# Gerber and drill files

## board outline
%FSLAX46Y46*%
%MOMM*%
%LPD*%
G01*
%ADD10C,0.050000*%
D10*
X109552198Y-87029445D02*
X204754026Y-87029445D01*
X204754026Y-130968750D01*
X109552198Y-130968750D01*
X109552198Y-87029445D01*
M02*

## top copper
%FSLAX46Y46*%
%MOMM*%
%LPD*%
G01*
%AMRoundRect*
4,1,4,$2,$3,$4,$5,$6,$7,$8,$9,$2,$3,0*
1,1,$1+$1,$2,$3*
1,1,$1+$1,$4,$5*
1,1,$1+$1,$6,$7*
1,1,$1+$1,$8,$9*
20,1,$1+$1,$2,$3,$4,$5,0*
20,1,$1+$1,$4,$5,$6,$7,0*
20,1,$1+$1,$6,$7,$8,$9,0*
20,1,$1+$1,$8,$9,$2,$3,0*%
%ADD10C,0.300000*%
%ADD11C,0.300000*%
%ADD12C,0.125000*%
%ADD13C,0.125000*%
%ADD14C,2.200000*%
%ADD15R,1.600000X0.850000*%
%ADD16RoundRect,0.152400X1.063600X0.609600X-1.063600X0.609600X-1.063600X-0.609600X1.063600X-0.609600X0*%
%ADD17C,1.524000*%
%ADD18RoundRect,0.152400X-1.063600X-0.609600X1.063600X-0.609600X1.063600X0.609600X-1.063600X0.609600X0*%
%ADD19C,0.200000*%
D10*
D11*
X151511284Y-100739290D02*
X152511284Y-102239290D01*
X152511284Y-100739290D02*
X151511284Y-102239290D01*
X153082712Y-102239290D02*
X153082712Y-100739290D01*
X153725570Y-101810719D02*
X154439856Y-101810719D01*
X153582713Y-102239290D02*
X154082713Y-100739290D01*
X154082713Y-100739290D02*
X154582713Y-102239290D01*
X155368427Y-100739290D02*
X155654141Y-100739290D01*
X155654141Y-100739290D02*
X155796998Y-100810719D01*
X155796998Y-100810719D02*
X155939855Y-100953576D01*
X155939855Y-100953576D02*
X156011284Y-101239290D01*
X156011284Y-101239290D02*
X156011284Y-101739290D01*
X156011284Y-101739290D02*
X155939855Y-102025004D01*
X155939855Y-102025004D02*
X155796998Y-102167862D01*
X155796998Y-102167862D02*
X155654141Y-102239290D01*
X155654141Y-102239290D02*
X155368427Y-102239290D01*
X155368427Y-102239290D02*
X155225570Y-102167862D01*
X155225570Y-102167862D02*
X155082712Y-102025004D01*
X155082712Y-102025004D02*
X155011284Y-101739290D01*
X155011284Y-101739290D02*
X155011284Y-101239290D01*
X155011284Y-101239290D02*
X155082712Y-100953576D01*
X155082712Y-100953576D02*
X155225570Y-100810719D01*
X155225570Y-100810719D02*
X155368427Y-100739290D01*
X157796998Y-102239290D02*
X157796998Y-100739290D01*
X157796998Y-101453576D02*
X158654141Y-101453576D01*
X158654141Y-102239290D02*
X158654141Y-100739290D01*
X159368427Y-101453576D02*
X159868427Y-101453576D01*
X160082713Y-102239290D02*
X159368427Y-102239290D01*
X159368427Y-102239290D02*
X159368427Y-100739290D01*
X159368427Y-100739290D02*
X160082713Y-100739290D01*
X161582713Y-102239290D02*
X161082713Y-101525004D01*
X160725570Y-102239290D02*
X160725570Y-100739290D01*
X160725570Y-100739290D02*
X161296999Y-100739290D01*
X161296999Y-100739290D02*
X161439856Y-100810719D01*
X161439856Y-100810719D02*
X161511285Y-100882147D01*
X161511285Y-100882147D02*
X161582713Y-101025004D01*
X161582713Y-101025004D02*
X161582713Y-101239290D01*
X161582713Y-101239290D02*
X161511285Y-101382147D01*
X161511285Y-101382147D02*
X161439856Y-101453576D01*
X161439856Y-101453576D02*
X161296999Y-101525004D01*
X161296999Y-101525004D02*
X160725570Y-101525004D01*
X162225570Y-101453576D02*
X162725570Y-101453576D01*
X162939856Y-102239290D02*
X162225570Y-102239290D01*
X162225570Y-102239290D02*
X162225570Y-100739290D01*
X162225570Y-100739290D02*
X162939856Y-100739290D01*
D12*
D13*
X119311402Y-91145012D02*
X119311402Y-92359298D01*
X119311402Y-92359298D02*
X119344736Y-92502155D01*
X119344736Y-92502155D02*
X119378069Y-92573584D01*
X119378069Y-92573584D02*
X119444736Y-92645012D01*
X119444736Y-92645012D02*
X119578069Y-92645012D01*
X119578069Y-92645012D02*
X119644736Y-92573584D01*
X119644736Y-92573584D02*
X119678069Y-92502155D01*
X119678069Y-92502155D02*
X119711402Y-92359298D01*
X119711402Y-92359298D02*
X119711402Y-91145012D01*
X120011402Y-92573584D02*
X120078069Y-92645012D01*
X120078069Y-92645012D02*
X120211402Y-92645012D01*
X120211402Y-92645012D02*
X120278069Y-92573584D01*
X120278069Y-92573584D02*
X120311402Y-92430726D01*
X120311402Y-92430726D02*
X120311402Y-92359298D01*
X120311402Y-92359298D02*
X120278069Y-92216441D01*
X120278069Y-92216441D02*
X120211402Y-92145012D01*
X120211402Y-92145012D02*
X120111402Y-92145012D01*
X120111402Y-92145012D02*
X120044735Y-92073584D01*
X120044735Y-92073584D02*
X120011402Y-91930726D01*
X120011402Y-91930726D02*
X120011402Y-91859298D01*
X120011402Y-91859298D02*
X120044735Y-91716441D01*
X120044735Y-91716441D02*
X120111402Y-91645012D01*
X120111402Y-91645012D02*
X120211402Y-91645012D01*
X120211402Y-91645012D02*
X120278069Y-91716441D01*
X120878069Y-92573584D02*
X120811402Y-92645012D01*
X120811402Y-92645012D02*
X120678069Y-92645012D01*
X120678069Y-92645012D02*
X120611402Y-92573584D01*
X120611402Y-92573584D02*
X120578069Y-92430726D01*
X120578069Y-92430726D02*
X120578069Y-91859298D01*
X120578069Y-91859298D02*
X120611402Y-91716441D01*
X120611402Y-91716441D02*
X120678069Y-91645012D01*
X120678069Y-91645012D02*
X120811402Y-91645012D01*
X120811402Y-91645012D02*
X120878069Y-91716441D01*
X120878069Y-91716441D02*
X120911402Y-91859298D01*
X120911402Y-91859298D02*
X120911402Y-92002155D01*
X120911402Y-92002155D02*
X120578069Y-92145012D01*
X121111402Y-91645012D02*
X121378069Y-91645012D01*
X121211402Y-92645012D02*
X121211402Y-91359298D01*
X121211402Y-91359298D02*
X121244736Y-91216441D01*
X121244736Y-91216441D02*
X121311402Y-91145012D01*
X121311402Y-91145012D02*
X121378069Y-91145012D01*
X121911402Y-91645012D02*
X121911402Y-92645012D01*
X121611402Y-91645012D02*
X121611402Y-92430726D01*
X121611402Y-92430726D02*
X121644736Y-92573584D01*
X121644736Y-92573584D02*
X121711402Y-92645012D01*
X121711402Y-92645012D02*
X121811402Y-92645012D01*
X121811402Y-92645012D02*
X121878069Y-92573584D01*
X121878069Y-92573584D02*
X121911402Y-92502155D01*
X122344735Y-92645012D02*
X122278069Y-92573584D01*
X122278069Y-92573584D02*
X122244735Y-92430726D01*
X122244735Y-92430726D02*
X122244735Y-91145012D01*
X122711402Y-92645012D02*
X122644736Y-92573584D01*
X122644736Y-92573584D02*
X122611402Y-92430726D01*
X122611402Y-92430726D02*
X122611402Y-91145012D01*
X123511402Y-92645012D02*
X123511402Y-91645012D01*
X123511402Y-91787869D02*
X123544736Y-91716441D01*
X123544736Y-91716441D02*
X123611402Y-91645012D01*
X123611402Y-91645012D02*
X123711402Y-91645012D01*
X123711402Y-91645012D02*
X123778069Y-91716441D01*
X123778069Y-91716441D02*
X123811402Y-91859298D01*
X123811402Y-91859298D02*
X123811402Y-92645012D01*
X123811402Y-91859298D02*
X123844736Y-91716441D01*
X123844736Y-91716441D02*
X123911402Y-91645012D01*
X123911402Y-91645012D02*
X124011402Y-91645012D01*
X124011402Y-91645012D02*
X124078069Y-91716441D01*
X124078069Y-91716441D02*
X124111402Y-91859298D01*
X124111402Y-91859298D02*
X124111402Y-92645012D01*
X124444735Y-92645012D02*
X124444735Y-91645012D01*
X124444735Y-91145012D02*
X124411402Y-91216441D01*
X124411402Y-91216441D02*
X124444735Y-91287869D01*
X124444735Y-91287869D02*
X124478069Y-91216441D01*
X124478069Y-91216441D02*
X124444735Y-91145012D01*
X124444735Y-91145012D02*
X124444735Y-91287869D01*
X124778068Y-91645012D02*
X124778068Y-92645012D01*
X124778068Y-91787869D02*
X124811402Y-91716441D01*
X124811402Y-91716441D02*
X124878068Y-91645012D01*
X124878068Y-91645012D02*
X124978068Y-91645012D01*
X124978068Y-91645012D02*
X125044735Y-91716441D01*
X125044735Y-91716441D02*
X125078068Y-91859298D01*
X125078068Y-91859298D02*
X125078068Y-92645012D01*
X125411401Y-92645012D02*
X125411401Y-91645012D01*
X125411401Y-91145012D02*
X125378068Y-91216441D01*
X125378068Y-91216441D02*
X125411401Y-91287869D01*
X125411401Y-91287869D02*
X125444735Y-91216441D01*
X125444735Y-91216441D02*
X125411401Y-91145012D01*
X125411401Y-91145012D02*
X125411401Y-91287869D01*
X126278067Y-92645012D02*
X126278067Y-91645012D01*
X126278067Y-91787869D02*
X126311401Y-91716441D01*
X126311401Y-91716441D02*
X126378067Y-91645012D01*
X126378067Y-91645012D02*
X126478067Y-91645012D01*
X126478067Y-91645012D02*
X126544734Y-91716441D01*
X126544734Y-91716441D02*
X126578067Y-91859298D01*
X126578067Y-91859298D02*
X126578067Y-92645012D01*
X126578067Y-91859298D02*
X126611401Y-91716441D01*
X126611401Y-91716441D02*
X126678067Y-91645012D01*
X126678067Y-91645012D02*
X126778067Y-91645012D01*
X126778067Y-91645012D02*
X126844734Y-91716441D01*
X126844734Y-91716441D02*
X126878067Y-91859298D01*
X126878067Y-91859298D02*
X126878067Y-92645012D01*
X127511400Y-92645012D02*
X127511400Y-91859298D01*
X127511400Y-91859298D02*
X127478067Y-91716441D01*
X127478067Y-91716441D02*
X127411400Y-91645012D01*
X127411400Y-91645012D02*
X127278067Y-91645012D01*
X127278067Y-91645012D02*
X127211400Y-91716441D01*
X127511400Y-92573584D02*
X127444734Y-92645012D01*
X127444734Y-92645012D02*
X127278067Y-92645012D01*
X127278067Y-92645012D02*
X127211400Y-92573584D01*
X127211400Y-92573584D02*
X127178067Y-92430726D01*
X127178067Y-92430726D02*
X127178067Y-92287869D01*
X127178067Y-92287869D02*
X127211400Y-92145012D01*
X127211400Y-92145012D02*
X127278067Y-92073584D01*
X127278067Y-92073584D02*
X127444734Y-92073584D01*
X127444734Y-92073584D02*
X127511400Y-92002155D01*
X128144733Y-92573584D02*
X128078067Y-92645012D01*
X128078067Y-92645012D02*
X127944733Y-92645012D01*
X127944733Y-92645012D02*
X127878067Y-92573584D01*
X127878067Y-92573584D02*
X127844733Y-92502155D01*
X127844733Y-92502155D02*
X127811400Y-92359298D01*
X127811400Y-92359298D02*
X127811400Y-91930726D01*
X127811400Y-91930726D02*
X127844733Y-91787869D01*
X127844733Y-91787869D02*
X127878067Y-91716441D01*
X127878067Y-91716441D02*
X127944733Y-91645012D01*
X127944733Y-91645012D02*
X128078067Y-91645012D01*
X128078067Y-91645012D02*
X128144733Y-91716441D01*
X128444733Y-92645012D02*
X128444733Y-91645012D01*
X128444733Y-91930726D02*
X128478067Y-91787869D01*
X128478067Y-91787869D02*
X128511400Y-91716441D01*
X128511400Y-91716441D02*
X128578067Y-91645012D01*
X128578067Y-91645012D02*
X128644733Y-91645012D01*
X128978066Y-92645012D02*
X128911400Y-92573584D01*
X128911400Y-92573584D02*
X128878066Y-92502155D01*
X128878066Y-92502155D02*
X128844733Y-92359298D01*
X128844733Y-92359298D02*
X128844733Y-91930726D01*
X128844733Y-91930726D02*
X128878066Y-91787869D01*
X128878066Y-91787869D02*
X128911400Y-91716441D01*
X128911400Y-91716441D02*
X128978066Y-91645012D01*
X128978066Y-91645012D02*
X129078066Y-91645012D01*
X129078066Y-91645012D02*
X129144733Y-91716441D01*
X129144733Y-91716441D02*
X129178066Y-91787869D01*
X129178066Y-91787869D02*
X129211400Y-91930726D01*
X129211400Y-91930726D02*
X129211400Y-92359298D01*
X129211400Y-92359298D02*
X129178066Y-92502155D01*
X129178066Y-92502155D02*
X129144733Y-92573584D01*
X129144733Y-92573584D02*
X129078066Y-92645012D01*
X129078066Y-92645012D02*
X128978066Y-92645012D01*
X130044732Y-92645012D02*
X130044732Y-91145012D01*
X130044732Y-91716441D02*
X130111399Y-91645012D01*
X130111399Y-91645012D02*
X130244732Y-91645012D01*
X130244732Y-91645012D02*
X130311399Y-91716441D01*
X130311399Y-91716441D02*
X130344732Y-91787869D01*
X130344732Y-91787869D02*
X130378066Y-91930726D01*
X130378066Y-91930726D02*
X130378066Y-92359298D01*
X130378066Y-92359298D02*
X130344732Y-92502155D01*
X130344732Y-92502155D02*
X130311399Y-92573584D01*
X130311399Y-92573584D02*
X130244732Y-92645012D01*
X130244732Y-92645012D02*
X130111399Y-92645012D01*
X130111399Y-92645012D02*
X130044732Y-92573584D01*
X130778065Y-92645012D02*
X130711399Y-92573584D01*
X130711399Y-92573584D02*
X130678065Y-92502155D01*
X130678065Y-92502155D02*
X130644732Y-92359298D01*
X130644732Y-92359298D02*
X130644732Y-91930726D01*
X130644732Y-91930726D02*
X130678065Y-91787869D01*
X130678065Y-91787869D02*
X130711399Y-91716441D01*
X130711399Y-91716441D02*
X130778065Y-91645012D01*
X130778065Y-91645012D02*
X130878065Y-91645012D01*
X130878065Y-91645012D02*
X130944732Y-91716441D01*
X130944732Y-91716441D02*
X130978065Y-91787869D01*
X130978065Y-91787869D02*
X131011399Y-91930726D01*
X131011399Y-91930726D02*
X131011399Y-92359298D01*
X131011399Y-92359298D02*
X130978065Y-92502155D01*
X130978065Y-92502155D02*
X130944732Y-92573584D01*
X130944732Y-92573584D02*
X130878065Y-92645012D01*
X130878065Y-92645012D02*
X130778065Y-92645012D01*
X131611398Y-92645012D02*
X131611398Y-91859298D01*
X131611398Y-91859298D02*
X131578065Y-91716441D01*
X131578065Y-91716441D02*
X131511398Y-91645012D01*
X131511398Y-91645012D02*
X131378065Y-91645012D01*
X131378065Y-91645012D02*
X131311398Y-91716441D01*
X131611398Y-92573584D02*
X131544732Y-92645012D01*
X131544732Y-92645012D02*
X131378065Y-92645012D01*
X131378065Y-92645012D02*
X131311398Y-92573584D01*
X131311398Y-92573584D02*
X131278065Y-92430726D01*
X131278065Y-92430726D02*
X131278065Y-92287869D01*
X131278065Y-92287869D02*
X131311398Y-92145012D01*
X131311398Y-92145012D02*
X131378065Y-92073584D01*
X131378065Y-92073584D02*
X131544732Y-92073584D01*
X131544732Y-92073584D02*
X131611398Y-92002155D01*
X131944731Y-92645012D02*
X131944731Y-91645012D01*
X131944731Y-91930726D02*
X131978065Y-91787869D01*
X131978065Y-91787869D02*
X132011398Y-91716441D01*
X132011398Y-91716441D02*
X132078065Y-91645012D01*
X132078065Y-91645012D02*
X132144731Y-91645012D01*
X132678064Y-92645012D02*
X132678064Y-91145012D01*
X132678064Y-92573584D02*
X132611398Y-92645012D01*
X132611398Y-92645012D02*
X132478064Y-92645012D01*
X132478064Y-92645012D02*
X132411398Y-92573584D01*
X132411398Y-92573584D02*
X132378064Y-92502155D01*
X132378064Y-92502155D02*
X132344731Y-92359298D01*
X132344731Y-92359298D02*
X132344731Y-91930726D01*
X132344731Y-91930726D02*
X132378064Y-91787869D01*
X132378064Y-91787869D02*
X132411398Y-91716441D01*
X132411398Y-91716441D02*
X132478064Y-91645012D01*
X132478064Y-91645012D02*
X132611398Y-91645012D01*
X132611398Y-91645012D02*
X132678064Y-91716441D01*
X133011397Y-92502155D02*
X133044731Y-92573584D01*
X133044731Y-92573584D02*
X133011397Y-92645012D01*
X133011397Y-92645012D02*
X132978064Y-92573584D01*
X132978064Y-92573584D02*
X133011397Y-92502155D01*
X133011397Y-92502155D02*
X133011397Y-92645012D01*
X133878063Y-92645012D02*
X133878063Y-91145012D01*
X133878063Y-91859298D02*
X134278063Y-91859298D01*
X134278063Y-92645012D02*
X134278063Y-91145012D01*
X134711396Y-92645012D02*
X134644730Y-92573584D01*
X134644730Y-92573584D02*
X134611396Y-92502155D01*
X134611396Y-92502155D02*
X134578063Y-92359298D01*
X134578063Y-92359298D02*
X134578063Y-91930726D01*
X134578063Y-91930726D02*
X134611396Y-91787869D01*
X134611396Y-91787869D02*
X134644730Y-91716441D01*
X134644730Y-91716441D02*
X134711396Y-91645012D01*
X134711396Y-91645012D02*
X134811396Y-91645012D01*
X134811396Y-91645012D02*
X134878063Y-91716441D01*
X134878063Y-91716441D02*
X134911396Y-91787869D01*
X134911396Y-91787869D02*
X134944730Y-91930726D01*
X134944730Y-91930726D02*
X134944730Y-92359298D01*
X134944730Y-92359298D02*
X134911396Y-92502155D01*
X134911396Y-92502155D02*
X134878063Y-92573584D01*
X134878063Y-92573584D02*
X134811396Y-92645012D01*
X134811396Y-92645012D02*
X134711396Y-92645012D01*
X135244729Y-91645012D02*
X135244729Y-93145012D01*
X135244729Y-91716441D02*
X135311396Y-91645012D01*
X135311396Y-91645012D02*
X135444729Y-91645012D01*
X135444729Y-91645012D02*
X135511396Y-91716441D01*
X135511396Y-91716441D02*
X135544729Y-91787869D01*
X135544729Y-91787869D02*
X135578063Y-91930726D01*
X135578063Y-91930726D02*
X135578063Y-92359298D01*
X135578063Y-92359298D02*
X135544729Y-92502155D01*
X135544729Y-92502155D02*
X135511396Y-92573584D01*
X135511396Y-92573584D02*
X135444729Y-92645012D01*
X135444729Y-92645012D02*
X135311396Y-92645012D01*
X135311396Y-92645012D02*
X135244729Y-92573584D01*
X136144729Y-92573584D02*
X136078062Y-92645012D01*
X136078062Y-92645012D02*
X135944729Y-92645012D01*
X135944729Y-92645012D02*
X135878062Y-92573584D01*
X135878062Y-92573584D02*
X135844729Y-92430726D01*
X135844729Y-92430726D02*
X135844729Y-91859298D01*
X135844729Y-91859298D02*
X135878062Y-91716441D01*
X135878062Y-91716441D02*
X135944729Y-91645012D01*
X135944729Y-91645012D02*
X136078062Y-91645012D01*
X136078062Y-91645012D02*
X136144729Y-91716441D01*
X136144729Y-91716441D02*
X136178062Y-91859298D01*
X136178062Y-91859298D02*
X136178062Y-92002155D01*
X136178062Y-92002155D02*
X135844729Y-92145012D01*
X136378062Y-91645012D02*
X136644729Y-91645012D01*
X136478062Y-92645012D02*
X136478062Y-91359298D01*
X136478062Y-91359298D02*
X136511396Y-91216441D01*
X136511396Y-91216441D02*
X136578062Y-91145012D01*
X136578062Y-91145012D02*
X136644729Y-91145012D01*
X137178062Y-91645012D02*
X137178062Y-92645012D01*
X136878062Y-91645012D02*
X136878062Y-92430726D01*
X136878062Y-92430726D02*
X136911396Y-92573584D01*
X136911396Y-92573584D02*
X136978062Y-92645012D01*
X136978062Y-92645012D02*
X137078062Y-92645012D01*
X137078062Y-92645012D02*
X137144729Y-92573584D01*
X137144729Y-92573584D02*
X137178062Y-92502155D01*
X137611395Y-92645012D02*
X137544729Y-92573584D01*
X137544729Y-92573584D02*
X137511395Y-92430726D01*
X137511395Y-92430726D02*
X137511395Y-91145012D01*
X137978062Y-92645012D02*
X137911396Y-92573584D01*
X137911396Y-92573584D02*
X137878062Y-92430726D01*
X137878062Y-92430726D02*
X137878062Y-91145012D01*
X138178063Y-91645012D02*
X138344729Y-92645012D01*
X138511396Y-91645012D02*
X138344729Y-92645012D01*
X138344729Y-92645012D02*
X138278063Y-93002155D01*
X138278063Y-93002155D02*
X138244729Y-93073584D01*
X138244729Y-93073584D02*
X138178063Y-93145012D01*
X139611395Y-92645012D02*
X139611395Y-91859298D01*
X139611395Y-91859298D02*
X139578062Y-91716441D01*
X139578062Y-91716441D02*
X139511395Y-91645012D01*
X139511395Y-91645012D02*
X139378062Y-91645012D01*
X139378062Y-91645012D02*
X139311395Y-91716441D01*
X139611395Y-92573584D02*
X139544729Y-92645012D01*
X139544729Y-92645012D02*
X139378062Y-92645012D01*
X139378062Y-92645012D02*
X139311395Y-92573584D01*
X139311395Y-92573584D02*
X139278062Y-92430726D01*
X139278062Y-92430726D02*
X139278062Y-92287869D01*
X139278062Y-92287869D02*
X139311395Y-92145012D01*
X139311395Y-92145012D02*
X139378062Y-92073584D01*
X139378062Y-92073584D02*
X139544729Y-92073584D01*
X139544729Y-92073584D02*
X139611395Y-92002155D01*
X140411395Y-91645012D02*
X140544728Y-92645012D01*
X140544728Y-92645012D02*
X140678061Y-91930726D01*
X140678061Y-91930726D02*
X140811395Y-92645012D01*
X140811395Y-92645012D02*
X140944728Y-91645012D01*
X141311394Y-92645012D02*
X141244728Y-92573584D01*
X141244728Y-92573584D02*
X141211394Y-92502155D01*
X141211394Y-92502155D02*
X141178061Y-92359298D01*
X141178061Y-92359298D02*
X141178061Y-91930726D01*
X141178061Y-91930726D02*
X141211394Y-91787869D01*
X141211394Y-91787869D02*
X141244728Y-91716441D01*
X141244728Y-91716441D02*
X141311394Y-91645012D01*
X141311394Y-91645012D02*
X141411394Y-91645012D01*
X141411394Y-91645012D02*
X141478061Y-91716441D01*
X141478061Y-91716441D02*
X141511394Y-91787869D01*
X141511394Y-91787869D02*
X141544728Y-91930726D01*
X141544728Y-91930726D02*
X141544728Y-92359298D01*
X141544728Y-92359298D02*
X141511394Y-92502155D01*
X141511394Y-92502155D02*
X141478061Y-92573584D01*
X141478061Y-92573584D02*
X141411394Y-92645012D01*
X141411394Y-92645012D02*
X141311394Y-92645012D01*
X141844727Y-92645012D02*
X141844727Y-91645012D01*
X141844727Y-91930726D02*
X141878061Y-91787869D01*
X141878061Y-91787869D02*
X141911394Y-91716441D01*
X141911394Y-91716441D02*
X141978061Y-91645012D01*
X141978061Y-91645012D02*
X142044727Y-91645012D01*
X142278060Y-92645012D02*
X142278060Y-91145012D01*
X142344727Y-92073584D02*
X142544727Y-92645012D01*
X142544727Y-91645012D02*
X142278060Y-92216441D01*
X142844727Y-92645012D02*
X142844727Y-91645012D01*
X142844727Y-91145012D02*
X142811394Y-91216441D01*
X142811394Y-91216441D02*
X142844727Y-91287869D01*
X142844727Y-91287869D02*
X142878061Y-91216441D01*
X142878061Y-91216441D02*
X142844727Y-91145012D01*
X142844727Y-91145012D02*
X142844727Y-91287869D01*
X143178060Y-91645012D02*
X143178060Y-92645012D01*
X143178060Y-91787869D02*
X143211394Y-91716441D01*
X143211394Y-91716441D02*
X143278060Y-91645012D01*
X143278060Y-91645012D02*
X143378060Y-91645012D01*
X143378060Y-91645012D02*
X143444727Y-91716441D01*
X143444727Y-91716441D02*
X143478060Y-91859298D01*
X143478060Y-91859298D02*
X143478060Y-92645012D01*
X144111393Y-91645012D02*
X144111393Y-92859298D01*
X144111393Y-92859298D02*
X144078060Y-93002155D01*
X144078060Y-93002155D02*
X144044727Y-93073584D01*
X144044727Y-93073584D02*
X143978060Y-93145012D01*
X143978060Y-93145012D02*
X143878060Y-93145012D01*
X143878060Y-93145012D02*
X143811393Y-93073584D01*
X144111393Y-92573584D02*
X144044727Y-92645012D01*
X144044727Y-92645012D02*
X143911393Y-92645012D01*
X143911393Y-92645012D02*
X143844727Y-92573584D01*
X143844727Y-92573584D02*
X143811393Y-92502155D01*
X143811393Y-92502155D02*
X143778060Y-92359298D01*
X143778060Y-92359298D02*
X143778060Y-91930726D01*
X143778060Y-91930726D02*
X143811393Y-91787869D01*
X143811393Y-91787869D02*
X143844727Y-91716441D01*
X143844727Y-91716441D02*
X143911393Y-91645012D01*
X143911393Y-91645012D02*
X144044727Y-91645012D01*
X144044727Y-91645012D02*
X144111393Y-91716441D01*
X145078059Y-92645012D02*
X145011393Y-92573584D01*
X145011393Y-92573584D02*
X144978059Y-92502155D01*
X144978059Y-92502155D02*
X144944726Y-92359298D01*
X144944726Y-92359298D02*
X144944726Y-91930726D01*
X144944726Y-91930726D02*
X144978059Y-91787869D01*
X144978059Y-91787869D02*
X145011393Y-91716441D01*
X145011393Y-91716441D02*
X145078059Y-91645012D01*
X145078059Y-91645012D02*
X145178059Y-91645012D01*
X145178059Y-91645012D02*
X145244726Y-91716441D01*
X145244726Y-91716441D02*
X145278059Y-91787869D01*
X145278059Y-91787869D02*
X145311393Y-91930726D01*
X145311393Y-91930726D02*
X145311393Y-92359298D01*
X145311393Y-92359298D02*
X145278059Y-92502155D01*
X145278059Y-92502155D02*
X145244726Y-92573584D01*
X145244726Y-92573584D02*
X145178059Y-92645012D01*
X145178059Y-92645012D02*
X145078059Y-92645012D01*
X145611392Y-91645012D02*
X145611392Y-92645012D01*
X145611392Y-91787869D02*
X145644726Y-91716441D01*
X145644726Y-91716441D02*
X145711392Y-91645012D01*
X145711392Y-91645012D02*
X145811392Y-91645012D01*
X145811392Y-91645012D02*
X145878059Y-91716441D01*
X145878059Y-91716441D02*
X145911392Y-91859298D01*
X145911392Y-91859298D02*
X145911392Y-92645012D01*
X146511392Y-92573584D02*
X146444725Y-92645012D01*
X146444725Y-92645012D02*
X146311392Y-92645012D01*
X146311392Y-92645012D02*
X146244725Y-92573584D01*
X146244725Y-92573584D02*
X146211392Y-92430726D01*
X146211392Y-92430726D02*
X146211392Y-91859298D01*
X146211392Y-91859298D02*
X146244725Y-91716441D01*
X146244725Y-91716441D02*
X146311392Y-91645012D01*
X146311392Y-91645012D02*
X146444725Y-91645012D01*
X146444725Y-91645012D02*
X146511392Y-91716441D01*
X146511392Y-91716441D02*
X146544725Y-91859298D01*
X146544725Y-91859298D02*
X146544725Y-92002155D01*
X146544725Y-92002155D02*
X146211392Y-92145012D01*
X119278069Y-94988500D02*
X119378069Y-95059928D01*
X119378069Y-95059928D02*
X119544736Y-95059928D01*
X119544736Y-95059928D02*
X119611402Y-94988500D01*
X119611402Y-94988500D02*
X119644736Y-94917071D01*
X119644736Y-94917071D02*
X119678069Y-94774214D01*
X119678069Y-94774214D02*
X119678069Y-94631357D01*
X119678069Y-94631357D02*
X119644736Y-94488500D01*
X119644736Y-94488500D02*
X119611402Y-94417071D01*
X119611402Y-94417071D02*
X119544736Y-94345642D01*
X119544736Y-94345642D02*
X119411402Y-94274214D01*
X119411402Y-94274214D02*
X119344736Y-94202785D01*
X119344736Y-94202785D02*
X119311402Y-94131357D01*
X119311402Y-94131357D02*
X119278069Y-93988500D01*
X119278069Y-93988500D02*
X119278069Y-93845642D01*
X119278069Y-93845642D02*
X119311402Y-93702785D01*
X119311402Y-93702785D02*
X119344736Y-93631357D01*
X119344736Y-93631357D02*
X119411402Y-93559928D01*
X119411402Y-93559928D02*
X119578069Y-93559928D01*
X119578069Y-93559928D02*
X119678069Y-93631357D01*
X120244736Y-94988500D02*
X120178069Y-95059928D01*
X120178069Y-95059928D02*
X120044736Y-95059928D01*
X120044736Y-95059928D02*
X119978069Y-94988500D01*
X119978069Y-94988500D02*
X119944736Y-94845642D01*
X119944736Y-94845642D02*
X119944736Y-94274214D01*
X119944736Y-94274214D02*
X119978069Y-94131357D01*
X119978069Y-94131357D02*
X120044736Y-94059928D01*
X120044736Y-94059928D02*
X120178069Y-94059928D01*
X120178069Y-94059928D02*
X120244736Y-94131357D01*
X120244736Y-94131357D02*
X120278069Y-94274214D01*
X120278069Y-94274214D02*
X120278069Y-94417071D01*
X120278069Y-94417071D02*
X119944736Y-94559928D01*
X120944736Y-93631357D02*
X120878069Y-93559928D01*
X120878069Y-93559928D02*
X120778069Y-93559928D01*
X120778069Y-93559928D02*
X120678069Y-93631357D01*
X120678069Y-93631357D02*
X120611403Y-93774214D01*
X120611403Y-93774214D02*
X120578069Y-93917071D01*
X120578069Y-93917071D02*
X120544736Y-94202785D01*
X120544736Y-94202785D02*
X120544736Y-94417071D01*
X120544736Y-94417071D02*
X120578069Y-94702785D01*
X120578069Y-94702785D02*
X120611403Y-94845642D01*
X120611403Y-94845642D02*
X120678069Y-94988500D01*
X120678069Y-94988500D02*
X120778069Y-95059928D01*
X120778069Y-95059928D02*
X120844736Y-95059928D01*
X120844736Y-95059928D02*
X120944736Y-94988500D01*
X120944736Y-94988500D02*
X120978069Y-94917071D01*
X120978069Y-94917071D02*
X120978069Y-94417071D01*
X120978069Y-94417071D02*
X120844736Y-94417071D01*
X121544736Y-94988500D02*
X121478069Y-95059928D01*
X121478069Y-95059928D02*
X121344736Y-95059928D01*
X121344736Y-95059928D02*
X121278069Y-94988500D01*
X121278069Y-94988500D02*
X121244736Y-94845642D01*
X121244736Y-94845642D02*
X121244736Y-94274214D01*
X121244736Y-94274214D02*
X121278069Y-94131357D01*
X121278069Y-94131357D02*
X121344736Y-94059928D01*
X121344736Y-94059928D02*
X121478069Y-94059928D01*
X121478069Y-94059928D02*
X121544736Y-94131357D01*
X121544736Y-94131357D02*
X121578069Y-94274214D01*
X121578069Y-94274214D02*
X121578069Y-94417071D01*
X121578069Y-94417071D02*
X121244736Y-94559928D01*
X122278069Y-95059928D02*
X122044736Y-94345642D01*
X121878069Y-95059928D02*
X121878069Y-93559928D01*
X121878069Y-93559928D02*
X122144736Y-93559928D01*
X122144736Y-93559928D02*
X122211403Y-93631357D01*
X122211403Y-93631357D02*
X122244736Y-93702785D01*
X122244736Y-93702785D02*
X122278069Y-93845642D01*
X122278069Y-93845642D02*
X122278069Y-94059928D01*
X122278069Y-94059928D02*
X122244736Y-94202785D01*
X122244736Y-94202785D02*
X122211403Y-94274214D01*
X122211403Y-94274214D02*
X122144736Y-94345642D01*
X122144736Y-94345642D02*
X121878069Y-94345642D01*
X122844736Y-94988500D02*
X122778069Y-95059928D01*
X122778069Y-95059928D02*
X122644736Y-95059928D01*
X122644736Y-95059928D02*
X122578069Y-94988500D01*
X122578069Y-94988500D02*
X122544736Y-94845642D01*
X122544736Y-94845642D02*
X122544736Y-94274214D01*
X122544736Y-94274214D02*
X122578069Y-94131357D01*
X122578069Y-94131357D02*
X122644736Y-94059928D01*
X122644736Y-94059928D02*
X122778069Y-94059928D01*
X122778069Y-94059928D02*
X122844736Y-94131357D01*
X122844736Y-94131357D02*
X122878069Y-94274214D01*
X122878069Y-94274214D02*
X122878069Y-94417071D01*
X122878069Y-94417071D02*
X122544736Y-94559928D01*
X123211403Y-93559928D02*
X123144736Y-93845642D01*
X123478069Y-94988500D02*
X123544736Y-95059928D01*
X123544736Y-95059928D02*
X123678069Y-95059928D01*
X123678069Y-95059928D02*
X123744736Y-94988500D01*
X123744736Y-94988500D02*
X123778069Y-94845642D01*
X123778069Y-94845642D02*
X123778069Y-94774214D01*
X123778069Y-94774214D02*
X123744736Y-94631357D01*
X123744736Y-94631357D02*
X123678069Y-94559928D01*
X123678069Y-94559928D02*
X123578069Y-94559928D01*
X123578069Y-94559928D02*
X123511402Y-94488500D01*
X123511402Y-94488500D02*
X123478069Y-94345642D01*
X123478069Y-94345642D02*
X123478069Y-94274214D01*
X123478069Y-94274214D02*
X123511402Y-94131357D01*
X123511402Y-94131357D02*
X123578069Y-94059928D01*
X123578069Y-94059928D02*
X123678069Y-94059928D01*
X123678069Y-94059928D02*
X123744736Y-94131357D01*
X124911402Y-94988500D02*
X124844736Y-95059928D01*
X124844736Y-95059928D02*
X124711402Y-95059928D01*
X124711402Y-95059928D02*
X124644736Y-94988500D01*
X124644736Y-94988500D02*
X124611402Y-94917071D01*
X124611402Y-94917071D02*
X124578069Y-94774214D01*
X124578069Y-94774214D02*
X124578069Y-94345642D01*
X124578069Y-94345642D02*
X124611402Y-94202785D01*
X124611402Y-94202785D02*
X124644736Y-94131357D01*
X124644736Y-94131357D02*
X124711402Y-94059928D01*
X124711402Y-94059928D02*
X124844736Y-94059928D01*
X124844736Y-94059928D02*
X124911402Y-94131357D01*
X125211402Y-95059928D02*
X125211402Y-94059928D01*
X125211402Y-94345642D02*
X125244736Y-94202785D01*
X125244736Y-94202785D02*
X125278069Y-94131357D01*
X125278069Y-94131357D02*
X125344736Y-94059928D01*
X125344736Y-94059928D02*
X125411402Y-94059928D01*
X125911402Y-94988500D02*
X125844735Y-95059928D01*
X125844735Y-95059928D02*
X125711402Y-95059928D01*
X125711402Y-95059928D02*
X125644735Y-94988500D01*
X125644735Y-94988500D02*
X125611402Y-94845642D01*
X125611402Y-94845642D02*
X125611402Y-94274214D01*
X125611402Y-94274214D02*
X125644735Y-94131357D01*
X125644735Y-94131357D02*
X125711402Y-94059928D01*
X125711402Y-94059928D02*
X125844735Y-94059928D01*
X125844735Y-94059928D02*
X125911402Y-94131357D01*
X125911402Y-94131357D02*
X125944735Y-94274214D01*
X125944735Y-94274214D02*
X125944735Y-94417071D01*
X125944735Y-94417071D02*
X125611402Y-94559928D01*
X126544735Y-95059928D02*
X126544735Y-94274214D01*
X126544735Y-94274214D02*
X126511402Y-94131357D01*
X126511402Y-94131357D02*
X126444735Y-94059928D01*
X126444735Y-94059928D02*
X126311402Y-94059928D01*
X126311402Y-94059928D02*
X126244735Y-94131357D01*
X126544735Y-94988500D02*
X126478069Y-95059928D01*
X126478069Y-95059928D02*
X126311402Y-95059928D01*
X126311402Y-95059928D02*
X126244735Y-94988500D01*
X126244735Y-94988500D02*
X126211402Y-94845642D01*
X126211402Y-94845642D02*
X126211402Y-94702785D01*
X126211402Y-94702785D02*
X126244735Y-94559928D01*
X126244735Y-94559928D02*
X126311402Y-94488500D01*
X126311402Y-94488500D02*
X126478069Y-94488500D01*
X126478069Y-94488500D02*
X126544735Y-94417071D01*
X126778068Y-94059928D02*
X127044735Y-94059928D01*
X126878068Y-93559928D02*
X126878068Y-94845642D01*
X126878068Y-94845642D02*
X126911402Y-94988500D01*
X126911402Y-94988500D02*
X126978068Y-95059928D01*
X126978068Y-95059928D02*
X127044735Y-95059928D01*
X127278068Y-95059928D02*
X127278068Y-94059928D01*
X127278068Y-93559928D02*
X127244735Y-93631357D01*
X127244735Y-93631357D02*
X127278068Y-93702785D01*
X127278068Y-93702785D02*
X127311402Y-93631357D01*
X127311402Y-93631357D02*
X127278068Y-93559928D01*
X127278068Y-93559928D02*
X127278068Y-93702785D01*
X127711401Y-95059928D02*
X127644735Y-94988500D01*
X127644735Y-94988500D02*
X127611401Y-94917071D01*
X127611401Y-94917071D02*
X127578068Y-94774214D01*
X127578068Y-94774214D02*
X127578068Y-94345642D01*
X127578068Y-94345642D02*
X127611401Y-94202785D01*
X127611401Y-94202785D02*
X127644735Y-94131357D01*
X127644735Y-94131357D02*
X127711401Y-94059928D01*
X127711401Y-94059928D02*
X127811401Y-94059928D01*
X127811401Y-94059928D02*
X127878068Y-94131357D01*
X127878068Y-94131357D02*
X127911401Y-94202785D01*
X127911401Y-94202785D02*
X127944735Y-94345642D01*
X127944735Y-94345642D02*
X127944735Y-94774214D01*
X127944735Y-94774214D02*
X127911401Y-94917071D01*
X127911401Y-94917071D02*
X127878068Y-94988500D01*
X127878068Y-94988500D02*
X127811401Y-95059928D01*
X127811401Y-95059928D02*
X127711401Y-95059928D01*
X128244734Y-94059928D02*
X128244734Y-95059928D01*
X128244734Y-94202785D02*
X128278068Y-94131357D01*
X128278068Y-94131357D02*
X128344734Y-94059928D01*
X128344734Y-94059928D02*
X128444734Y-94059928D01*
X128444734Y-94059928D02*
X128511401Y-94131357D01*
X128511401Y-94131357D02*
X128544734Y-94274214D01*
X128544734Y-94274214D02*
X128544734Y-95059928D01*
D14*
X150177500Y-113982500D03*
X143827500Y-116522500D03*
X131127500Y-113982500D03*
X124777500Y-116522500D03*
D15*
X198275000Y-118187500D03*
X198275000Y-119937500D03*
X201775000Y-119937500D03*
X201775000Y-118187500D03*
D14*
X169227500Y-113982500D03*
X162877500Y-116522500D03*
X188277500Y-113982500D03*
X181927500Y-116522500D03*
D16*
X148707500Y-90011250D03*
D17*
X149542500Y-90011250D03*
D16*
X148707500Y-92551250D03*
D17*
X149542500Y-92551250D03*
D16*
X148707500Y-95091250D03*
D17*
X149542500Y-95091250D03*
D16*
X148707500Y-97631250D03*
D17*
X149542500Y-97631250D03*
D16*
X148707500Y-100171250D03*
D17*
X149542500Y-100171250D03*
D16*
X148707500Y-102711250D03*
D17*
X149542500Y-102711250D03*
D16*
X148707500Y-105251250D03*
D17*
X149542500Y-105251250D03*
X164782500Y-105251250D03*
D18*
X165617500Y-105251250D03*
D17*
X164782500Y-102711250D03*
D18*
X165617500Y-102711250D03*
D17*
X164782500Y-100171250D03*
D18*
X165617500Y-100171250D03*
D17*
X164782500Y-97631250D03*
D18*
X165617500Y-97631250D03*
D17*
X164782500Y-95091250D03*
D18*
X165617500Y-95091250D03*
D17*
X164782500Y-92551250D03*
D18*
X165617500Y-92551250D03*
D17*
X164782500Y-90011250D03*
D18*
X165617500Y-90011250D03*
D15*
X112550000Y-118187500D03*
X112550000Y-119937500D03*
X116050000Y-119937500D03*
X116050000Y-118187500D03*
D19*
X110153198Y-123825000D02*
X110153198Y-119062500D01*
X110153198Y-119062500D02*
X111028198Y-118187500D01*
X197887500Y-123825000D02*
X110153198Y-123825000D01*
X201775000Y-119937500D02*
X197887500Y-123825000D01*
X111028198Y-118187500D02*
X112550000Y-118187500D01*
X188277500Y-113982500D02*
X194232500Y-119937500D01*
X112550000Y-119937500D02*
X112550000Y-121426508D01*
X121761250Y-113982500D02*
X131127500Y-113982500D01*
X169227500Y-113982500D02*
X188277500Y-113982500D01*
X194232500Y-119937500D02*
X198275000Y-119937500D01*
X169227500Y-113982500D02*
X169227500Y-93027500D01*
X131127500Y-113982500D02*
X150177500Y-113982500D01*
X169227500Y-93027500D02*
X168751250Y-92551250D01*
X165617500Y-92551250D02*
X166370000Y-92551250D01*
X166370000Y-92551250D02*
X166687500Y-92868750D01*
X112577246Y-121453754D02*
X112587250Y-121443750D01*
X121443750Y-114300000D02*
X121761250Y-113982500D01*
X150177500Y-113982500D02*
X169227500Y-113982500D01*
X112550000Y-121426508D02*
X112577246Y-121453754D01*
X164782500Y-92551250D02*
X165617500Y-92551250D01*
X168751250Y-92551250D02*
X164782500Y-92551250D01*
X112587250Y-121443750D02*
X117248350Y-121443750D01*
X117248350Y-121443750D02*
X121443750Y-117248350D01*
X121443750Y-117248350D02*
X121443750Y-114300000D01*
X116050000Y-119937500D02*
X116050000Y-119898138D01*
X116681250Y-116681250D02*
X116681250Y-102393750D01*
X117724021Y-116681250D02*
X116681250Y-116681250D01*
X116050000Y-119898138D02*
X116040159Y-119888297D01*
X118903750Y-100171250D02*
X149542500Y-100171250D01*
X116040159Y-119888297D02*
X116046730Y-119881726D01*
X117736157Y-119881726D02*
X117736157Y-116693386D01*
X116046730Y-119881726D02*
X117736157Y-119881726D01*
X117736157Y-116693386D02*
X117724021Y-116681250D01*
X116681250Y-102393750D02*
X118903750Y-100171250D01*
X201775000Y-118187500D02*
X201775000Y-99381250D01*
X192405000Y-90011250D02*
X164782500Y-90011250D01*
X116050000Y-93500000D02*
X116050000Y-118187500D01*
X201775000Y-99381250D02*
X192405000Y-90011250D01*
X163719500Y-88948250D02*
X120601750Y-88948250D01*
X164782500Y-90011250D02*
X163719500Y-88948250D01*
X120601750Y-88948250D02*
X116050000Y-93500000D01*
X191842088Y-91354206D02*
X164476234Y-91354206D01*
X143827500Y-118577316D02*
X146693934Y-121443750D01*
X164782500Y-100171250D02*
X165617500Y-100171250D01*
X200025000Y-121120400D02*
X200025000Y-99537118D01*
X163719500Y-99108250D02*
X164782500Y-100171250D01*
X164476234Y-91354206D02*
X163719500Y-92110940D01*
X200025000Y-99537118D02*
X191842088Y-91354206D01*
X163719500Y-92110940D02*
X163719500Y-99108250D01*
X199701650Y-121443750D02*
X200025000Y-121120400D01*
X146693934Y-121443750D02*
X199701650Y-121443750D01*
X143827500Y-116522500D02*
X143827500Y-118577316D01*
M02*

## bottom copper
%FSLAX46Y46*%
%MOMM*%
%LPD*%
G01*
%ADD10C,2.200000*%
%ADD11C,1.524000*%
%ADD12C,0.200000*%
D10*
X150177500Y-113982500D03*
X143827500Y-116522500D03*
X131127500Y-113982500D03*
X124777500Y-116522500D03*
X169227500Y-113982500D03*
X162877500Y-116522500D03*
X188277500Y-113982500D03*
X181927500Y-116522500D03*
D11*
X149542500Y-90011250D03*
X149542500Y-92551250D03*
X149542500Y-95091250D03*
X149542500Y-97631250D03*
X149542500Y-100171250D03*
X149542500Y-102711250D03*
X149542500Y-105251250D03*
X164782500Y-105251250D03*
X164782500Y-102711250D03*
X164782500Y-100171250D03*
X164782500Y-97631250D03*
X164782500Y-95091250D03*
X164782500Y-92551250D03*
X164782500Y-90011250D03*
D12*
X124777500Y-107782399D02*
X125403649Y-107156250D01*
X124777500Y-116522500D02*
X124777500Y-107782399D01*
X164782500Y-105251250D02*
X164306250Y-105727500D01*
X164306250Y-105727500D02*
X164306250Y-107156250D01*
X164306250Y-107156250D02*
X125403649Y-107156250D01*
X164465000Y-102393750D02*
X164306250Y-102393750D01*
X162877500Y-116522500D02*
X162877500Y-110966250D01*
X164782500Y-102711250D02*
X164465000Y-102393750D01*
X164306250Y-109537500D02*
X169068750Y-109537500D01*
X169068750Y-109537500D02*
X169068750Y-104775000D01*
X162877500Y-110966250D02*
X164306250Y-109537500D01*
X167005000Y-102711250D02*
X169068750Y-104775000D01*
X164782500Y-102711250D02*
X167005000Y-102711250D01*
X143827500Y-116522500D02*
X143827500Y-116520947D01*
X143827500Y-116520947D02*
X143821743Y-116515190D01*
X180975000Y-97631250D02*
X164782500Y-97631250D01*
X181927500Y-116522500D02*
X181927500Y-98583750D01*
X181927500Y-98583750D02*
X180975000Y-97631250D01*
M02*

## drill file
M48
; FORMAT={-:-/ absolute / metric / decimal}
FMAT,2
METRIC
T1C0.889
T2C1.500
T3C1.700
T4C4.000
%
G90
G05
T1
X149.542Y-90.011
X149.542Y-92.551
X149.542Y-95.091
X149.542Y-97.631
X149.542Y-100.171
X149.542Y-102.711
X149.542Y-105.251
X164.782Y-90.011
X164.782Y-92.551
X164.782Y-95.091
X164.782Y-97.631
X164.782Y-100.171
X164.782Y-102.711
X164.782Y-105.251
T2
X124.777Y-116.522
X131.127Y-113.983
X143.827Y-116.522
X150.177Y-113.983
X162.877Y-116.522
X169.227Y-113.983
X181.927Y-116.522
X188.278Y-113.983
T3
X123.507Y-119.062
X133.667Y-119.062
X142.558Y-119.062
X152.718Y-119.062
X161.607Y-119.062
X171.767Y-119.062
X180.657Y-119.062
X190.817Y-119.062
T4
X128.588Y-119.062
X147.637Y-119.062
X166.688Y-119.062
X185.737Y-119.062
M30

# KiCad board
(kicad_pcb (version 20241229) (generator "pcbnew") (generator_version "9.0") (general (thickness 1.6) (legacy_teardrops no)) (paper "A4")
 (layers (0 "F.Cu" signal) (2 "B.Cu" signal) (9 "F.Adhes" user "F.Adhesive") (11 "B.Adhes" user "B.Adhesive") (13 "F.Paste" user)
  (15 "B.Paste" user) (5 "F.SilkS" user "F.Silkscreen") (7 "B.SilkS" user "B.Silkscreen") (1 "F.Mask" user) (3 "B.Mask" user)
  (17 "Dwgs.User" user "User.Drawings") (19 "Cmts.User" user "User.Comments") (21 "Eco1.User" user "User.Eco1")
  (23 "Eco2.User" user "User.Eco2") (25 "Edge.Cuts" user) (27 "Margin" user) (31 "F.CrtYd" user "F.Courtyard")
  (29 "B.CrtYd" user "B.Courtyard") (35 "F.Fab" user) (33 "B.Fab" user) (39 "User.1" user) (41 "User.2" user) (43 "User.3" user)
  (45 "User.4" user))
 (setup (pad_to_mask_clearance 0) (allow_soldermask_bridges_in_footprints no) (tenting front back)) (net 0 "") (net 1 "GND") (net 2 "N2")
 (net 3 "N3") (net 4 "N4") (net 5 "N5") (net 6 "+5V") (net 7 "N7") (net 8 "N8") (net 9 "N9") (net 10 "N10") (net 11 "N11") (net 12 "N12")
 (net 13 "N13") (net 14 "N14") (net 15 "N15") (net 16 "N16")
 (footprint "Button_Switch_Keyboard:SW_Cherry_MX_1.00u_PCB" (layer "F.Cu") (at 150.1775 113.9825)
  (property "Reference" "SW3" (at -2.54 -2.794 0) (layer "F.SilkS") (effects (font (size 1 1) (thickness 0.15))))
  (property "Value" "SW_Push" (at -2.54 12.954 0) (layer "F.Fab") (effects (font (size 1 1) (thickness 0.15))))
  (pad "" np_thru_hole circle (at -7.62 5.08) (size 1.7 1.7) (drill 1.7) (layers "*.Cu" "*.Mask"))
  (pad "" np_thru_hole circle (at -2.54 5.08) (size 4 4) (drill 4) (layers "*.Cu" "*.Mask"))
  (pad "" np_thru_hole circle (at 2.54 5.08) (size 1.7 1.7) (drill 1.7) (layers "*.Cu" "*.Mask"))
  (pad "1" thru_hole circle (at 0 0) (size 2.2 2.2) (drill 1.5) (layers "*.Cu" "*.Mask") (remove_unused_layers no) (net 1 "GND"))
  (pad "2" thru_hole circle (at -6.35 2.54) (size 2.2 2.2) (drill 1.5) (layers "*.Cu" "*.Mask") (remove_unused_layers no) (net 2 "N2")))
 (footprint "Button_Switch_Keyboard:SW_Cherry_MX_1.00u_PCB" (layer "F.Cu") (at 131.1275 113.9825)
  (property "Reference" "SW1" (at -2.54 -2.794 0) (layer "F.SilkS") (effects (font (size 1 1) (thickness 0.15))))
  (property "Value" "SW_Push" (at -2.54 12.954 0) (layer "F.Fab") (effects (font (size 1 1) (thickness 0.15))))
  (pad "" np_thru_hole circle (at -7.62 5.08) (size 1.7 1.7) (drill 1.7) (layers "*.Cu" "*.Mask"))
  (pad "" np_thru_hole circle (at -2.54 5.08) (size 4 4) (drill 4) (layers "*.Cu" "*.Mask"))
  (pad "" np_thru_hole circle (at 2.54 5.08) (size 1.7 1.7) (drill 1.7) (layers "*.Cu" "*.Mask"))
  (pad "1" thru_hole circle (at 0 0) (size 2.2 2.2) (drill 1.5) (layers "*.Cu" "*.Mask") (remove_unused_layers no) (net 1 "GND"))
  (pad "2" thru_hole circle (at -6.35 2.54) (size 2.2 2.2) (drill 1.5) (layers "*.Cu" "*.Mask") (remove_unused_layers no) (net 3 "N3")))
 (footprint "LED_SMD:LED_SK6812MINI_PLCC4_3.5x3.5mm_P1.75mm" (layer "F.Cu") (at 200.025 119.0625)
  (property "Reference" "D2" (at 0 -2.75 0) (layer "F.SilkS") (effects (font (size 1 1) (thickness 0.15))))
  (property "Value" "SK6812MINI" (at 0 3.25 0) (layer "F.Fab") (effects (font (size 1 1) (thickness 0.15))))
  (pad "1" smd rect (at -1.75 -0.875) (size 1.6 0.85) (layers "F.Cu" "F.Mask" "F.Paste") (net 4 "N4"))
  (pad "2" smd rect (at -1.75 0.875) (size 1.6 0.85) (layers "F.Cu" "F.Mask" "F.Paste") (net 1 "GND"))
  (pad "3" smd rect (at 1.75 0.875) (size 1.6 0.85) (layers "F.Cu" "F.Mask" "F.Paste") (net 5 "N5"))
  (pad "4" smd rect (at 1.75 -0.875) (size 1.6 0.85) (layers "F.Cu" "F.Mask" "F.Paste") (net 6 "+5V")))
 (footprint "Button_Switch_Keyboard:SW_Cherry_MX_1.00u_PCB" (layer "F.Cu") (at 169.2275 113.9825)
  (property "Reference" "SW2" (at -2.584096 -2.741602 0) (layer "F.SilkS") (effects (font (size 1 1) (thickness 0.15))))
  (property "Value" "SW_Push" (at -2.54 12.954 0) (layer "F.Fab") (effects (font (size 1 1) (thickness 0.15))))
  (pad "" np_thru_hole circle (at -7.62 5.08) (size 1.7 1.7) (drill 1.7) (layers "*.Cu" "*.Mask"))
  (pad "" np_thru_hole circle (at -2.54 5.08) (size 4 4) (drill 4) (layers "*.Cu" "*.Mask"))
  (pad "" np_thru_hole circle (at 2.54 5.08) (size 1.7 1.7) (drill 1.7) (layers "*.Cu" "*.Mask"))
  (pad "1" thru_hole circle (at 0 0) (size 2.2 2.2) (drill 1.5) (layers "*.Cu" "*.Mask") (remove_unused_layers no) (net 1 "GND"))
  (pad "2" thru_hole circle (at -6.35 2.54) (size 2.2 2.2) (drill 1.5) (layers "*.Cu" "*.Mask") (remove_unused_layers no) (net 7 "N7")))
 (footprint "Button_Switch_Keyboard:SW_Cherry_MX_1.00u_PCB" (layer "F.Cu") (at 188.2775 113.9825)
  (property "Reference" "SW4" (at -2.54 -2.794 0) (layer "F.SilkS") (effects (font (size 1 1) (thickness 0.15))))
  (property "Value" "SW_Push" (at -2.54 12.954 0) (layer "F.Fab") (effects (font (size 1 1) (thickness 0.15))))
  (pad "" np_thru_hole circle (at -7.62 5.08) (size 1.7 1.7) (drill 1.7) (layers "*.Cu" "*.Mask"))
  (pad "" np_thru_hole circle (at -2.54 5.08) (size 4 4) (drill 4) (layers "*.Cu" "*.Mask"))
  (pad "" np_thru_hole circle (at 2.54 5.08) (size 1.7 1.7) (drill 1.7) (layers "*.Cu" "*.Mask"))
  (pad "1" thru_hole circle (at 0 0) (size 2.2 2.2) (drill 1.5) (layers "*.Cu" "*.Mask") (remove_unused_layers no) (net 1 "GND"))
  (pad "2" thru_hole circle (at -6.35 2.54) (size 2.2 2.2) (drill 1.5) (layers "*.Cu" "*.Mask") (remove_unused_layers no) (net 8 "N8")))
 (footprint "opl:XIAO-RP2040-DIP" (layer "F.Cu") (at 157.1625 97.63125)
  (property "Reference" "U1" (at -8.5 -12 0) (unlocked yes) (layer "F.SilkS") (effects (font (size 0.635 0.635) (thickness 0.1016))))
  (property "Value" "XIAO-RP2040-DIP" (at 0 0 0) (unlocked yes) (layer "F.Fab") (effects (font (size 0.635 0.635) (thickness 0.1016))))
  (pad "1" smd roundrect (at -8.455 -7.62 180) (size 2.432 1.524) (layers "F.Cu" "F.Mask") (roundrect_rratio 0.1) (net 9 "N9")
   (thermal_bridge_angle 45))
  (pad "1" thru_hole circle (at -7.62 -7.62 180) (size 1.524 1.524) (drill 0.889) (layers "*.Cu" "*.Mask") (remove_unused_layers no)
   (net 9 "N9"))
  (pad "2" smd roundrect (at -8.455 -5.08 180) (size 2.432 1.524) (layers "F.Cu" "F.Mask") (roundrect_rratio 0.1) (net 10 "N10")
   (thermal_bridge_angle 45))
  (pad "2" thru_hole circle (at -7.62 -5.08 180) (size 1.524 1.524) (drill 0.889) (layers "*.Cu" "*.Mask") (remove_unused_layers no)
   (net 10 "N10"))
  (pad "3" smd roundrect (at -8.455 -2.54 180) (size 2.432 1.524) (layers "F.Cu" "F.Mask") (roundrect_rratio 0.1) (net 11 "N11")
   (thermal_bridge_angle 45))
  (pad "3" thru_hole circle (at -7.62 -2.54 180) (size 1.524 1.524) (drill 0.889) (layers "*.Cu" "*.Mask") (remove_unused_layers no)
   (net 11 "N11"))
  (pad "4" smd roundrect (at -8.455 0 180) (size 2.432 1.524) (layers "F.Cu" "F.Mask") (roundrect_rratio 0.1) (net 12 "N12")
   (thermal_bridge_angle 45))
  (pad "4" thru_hole circle (at -7.62 0 180) (size 1.524 1.524) (drill 0.889) (layers "*.Cu" "*.Mask") (remove_unused_layers no)
   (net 12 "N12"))
  (pad "5" smd roundrect (at -8.455 2.54 180) (size 2.432 1.524) (layers "F.Cu" "F.Mask") (roundrect_rratio 0.1) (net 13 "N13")
   (thermal_bridge_angle 45))
  (pad "5" thru_hole circle (at -7.62 2.54 180) (size 1.524 1.524) (drill 0.889) (layers "*.Cu" "*.Mask") (remove_unused_layers no)
   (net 13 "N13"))
  (pad "6" smd roundrect (at -8.455 5.08 180) (size 2.432 1.524) (layers "F.Cu" "F.Mask") (roundrect_rratio 0.1) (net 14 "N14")
   (thermal_bridge_angle 45))
  (pad "6" thru_hole circle (at -7.62 5.08 180) (size 1.524 1.524) (drill 0.889) (layers "*.Cu" "*.Mask") (remove_unused_layers no)
   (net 14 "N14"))
  (pad "7" smd roundrect (at -8.455 7.62 180) (size 2.432 1.524) (layers "F.Cu" "F.Mask") (roundrect_rratio 0.1) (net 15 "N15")
   (thermal_bridge_angle 45))
  (pad "7" thru_hole circle (at -7.62 7.62 180) (size 1.524 1.524) (drill 0.889) (layers "*.Cu" "*.Mask") (remove_unused_layers no)
   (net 15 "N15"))
  (pad "8" thru_hole circle (at 7.62 7.62) (size 1.524 1.524) (drill 0.889) (layers "*.Cu" "*.Mask") (remove_unused_layers no) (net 3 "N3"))
  (pad "8" smd roundrect (at 8.455 7.62) (size 2.432 1.524) (layers "F.Cu" "F.Mask") (roundrect_rratio 0.1) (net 3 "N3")
   (thermal_bridge_angle 45))
  (pad "9" thru_hole circle (at 7.62 5.08) (size 1.524 1.524) (drill 0.889) (layers "*.Cu" "*.Mask") (remove_unused_layers no) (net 7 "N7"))
  (pad "9" smd roundrect (at 8.455 5.08) (size 2.432 1.524) (layers "F.Cu" "F.Mask") (roundrect_rratio 0.1) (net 7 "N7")
   (thermal_bridge_angle 45))
  (pad "10" thru_hole circle (at 7.62 2.54) (size 1.524 1.524) (drill 0.889) (layers "*.Cu" "*.Mask") (remove_unused_layers no) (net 2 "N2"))
  (pad "10" smd roundrect (at 8.455 2.54) (size 2.432 1.524) (layers "F.Cu" "F.Mask") (roundrect_rratio 0.1) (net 2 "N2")
   (thermal_bridge_angle 45))
  (pad "11" thru_hole circle (at 7.62 0) (size 1.524 1.524) (drill 0.889) (layers "*.Cu" "*.Mask") (remove_unused_layers no) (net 8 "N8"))
  (pad "11" smd roundrect (at 8.455 0) (size 2.432 1.524) (layers "F.Cu" "F.Mask") (roundrect_rratio 0.1) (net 8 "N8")
   (thermal_bridge_angle 45))
  (pad "12" thru_hole circle (at 7.62 -2.54) (size 1.524 1.524) (drill 0.889) (layers "*.Cu" "*.Mask") (remove_unused_layers no)
   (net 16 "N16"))
  (pad "12" smd roundrect (at 8.455 -2.54) (size 2.432 1.524) (layers "F.Cu" "F.Mask") (roundrect_rratio 0.1) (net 16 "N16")
   (thermal_bridge_angle 45))
  (pad "13" thru_hole circle (at 7.62 -5.08) (size 1.524 1.524) (drill 0.889) (layers "*.Cu" "*.Mask") (remove_unused_layers no)
   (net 1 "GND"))
  (pad "13" smd roundrect (at 8.455 -5.08) (size 2.432 1.524) (layers "F.Cu" "F.Mask") (roundrect_rratio 0.1) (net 1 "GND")
   (thermal_bridge_angle 45))
  (pad "14" thru_hole circle (at 7.62 -7.62) (size 1.524 1.524) (drill 0.889) (layers "*.Cu" "*.Mask") (remove_unused_layers no)
   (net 6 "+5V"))
  (pad "14" smd roundrect (at 8.455 -7.62) (size 2.432 1.524) (layers "F.Cu" "F.Mask") (roundrect_rratio 0.1) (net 6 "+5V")
   (thermal_bridge_angle 45)))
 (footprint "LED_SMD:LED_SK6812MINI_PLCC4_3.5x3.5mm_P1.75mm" (layer "F.Cu") (at 114.3 119.0625)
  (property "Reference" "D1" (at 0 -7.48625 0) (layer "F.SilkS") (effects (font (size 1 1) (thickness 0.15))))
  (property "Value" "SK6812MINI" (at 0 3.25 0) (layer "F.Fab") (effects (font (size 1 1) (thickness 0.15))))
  (pad "1" smd rect (at -1.75 -0.875) (size 1.6 0.85) (layers "F.Cu" "F.Mask" "F.Paste") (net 5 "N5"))
  (pad "2" smd rect (at -1.75 0.875) (size 1.6 0.85) (layers "F.Cu" "F.Mask" "F.Paste") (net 1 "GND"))
  (pad "3" smd rect (at 1.75 0.875) (size 1.6 0.85) (layers "F.Cu" "F.Mask" "F.Paste") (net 13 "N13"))
  (pad "4" smd rect (at 1.75 -0.875) (size 1.6 0.85) (layers "F.Cu" "F.Mask" "F.Paste") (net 6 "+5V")))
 (gr_rect (start 109.552198 87.029445) (end 204.754026 130.96875) (stroke (width 0.05) (type default)) (fill no) (layer "Edge.Cuts"))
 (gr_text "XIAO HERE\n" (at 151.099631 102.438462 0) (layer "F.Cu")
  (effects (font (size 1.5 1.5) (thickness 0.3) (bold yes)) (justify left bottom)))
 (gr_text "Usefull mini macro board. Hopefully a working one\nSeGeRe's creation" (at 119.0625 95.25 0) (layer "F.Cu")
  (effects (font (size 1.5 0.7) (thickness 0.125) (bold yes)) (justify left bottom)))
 (segment (start 110.153198 123.825) (end 110.153198 119.0625) (width 0.2) (layer "F.Cu") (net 5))
 (segment (start 110.153198 119.0625) (end 111.028198 118.1875) (width 0.2) (layer "F.Cu") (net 5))
 (segment (start 197.8875 123.825) (end 110.153198 123.825) (width 0.2) (layer "F.Cu") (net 5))
 (segment (start 201.775 119.9375) (end 197.8875 123.825) (width 0.2) (layer "F.Cu") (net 5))
 (segment (start 111.028198 118.1875) (end 112.55 118.1875) (width 0.2) (layer "F.Cu") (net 5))
 (segment (start 188.2775 113.9825) (end 194.2325 119.9375) (width 0.2) (layer "F.Cu") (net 1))
 (segment (start 112.55 119.9375) (end 112.55 121.426508) (width 0.2) (layer "F.Cu") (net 1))
 (segment (start 121.76125 113.9825) (end 131.1275 113.9825) (width 0.2) (layer "F.Cu") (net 1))
 (segment (start 169.2275 113.9825) (end 188.2775 113.9825) (width 0.2) (layer "F.Cu") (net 1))
 (segment (start 194.2325 119.9375) (end 198.275 119.9375) (width 0.2) (layer "F.Cu") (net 1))
 (segment (start 169.2275 113.9825) (end 169.2275 93.0275) (width 0.2) (layer "F.Cu") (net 1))
 (segment (start 131.1275 113.9825) (end 150.1775 113.9825) (width 0.2) (layer "F.Cu") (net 1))
 (segment (start 169.2275 93.0275) (end 168.75125 92.55125) (width 0.2) (layer "F.Cu") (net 1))
 (segment (start 165.6175 92.55125) (end 166.37 92.55125) (width 0.2) (layer "F.Cu") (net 1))
 (segment (start 166.37 92.55125) (end 166.6875 92.86875) (width 0.2) (layer "F.Cu") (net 1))
 (segment (start 112.577246 121.453754) (end 112.58725 121.44375) (width 0.2) (layer "F.Cu") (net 1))
 (segment (start 121.44375 114.3) (end 121.76125 113.9825) (width 0.2) (layer "F.Cu") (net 1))
 (segment (start 150.1775 113.9825) (end 169.2275 113.9825) (width 0.2) (layer "F.Cu") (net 1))
 (segment (start 112.55 121.426508) (end 112.577246 121.453754) (width 0.2) (layer "F.Cu") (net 1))
 (segment (start 164.7825 92.55125) (end 165.6175 92.55125) (width 0.2) (layer "F.Cu") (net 1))
 (segment (start 168.75125 92.55125) (end 164.7825 92.55125) (width 0.2) (layer "F.Cu") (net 1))
 (segment (start 112.58725 121.44375) (end 117.24835 121.44375) (width 0.2) (layer "F.Cu") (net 1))
 (segment (start 117.24835 121.44375) (end 121.44375 117.24835) (width 0.2) (layer "F.Cu") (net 1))
 (segment (start 121.44375 117.24835) (end 121.44375 114.3) (width 0.2) (layer "F.Cu") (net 1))
 (segment (start 116.05 119.9375) (end 116.05 119.898138) (width 0.2) (layer "F.Cu") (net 13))
 (segment (start 116.68125 116.68125) (end 116.68125 102.39375) (width 0.2) (layer "F.Cu") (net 13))
 (segment (start 117.724021 116.68125) (end 116.68125 116.68125) (width 0.2) (layer "F.Cu") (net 13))
 (segment (start 116.05 119.898138) (end 116.040159 119.888297) (width 0.2) (layer "F.Cu") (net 13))
 (segment (start 118.90375 100.17125) (end 149.5425 100.17125) (width 0.2) (layer "F.Cu") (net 13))
 (segment (start 116.040159 119.888297) (end 116.04673 119.881726) (width 0.2) (layer "F.Cu") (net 13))
 (segment (start 117.736157 119.881726) (end 117.736157 116.693386) (width 0.2) (layer "F.Cu") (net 13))
 (segment (start 116.04673 119.881726) (end 117.736157 119.881726) (width 0.2) (layer "F.Cu") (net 13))
 (segment (start 117.736157 116.693386) (end 117.724021 116.68125) (width 0.2) (layer "F.Cu") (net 13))
 (segment (start 116.68125 102.39375) (end 118.90375 100.17125) (width 0.2) (layer "F.Cu") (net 13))
 (segment (start 201.775 118.1875) (end 201.775 99.38125) (width 0.2) (layer "F.Cu") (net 6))
 (segment (start 192.405 90.01125) (end 164.7825 90.01125) (width 0.2) (layer "F.Cu") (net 6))
 (segment (start 116.05 93.5) (end 116.05 118.1875) (width 0.2) (layer "F.Cu") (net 6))
 (segment (start 201.775 99.38125) (end 192.405 90.01125) (width 0.2) (layer "F.Cu") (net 6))
 (segment (start 163.7195 88.94825) (end 120.60175 88.94825) (width 0.2) (layer "F.Cu") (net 6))
 (segment (start 164.7825 90.01125) (end 163.7195 88.94825) (width 0.2) (layer "F.Cu") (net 6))
 (segment (start 120.60175 88.94825) (end 116.05 93.5) (width 0.2) (layer "F.Cu") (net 6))
 (segment (start 124.7775 107.782399) (end 125.403649 107.15625) (width 0.2) (layer "B.Cu") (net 3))
 (segment (start 124.7775 116.5225) (end 124.7775 107.782399) (width 0.2) (layer "B.Cu") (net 3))
 (segment (start 164.7825 105.25125) (end 164.30625 105.7275) (width 0.2) (layer "B.Cu") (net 3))
 (segment (start 164.30625 105.7275) (end 164.30625 107.15625) (width 0.2) (layer "B.Cu") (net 3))
 (segment (start 164.30625 107.15625) (end 125.403649 107.15625) (width 0.2) (layer "B.Cu") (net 3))
 (segment (start 164.465 102.39375) (end 164.30625 102.39375) (width 0.2) (layer "B.Cu") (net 7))
 (segment (start 162.8775 116.5225) (end 162.8775 110.96625) (width 0.2) (layer "B.Cu") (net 7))
 (segment (start 164.7825 102.71125) (end 164.465 102.39375) (width 0.2) (layer "B.Cu") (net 7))
 (segment (start 164.30625 109.5375) (end 169.06875 109.5375) (width 0.2) (layer "B.Cu") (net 7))
 (segment (start 169.06875 109.5375) (end 169.06875 104.775) (width 0.2) (layer "B.Cu") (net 7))
 (segment (start 162.8775 110.96625) (end 164.30625 109.5375) (width 0.2) (layer "B.Cu") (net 7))
 (segment (start 167.005 102.71125) (end 169.06875 104.775) (width 0.2) (layer "B.Cu") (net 7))
 (segment (start 164.7825 102.71125) (end 167.005 102.71125) (width 0.2) (layer "B.Cu") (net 7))
 (segment (start 191.842088 91.354206) (end 164.476234 91.354206) (width 0.2) (layer "F.Cu") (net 2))
 (segment (start 143.8275 118.577316) (end 146.693934 121.44375) (width 0.2) (layer "F.Cu") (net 2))
 (segment (start 164.7825 100.17125) (end 165.6175 100.17125) (width 0.2) (layer "F.Cu") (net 2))
 (segment (start 200.025 121.1204) (end 200.025 99.537118) (width 0.2) (layer "F.Cu") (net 2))
 (segment (start 163.7195 99.10825) (end 164.7825 100.17125) (width 0.2) (layer "F.Cu") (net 2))
 (segment (start 164.476234 91.354206) (end 163.7195 92.11094) (width 0.2) (layer "F.Cu") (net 2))
 (segment (start 200.025 99.537118) (end 191.842088 91.354206) (width 0.2) (layer "F.Cu") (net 2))
 (segment (start 163.7195 92.11094) (end 163.7195 99.10825) (width 0.2) (layer "F.Cu") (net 2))
 (segment (start 199.70165 121.44375) (end 200.025 121.1204) (width 0.2) (layer "F.Cu") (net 2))
 (segment (start 146.693934 121.44375) (end 199.70165 121.44375) (width 0.2) (layer "F.Cu") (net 2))
 (segment (start 143.8275 116.5225) (end 143.8275 118.577316) (width 0.2) (layer "F.Cu") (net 2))
 (segment (start 143.8275 116.5225) (end 143.8275 116.520947) (width 0.2) (layer "B.Cu") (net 2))
 (segment (start 143.8275 116.520947) (end 143.821743 116.51519) (width 0.2) (layer "B.Cu") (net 2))
 (segment (start 180.975 97.63125) (end 164.7825 97.63125) (width 0.2) (layer "B.Cu") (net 8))
 (segment (start 181.9275 116.5225) (end 181.9275 98.58375) (width 0.2) (layer "B.Cu") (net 8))
 (segment (start 181.9275 98.58375) (end 180.975 97.63125) (width 0.2) (layer "B.Cu") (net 8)))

